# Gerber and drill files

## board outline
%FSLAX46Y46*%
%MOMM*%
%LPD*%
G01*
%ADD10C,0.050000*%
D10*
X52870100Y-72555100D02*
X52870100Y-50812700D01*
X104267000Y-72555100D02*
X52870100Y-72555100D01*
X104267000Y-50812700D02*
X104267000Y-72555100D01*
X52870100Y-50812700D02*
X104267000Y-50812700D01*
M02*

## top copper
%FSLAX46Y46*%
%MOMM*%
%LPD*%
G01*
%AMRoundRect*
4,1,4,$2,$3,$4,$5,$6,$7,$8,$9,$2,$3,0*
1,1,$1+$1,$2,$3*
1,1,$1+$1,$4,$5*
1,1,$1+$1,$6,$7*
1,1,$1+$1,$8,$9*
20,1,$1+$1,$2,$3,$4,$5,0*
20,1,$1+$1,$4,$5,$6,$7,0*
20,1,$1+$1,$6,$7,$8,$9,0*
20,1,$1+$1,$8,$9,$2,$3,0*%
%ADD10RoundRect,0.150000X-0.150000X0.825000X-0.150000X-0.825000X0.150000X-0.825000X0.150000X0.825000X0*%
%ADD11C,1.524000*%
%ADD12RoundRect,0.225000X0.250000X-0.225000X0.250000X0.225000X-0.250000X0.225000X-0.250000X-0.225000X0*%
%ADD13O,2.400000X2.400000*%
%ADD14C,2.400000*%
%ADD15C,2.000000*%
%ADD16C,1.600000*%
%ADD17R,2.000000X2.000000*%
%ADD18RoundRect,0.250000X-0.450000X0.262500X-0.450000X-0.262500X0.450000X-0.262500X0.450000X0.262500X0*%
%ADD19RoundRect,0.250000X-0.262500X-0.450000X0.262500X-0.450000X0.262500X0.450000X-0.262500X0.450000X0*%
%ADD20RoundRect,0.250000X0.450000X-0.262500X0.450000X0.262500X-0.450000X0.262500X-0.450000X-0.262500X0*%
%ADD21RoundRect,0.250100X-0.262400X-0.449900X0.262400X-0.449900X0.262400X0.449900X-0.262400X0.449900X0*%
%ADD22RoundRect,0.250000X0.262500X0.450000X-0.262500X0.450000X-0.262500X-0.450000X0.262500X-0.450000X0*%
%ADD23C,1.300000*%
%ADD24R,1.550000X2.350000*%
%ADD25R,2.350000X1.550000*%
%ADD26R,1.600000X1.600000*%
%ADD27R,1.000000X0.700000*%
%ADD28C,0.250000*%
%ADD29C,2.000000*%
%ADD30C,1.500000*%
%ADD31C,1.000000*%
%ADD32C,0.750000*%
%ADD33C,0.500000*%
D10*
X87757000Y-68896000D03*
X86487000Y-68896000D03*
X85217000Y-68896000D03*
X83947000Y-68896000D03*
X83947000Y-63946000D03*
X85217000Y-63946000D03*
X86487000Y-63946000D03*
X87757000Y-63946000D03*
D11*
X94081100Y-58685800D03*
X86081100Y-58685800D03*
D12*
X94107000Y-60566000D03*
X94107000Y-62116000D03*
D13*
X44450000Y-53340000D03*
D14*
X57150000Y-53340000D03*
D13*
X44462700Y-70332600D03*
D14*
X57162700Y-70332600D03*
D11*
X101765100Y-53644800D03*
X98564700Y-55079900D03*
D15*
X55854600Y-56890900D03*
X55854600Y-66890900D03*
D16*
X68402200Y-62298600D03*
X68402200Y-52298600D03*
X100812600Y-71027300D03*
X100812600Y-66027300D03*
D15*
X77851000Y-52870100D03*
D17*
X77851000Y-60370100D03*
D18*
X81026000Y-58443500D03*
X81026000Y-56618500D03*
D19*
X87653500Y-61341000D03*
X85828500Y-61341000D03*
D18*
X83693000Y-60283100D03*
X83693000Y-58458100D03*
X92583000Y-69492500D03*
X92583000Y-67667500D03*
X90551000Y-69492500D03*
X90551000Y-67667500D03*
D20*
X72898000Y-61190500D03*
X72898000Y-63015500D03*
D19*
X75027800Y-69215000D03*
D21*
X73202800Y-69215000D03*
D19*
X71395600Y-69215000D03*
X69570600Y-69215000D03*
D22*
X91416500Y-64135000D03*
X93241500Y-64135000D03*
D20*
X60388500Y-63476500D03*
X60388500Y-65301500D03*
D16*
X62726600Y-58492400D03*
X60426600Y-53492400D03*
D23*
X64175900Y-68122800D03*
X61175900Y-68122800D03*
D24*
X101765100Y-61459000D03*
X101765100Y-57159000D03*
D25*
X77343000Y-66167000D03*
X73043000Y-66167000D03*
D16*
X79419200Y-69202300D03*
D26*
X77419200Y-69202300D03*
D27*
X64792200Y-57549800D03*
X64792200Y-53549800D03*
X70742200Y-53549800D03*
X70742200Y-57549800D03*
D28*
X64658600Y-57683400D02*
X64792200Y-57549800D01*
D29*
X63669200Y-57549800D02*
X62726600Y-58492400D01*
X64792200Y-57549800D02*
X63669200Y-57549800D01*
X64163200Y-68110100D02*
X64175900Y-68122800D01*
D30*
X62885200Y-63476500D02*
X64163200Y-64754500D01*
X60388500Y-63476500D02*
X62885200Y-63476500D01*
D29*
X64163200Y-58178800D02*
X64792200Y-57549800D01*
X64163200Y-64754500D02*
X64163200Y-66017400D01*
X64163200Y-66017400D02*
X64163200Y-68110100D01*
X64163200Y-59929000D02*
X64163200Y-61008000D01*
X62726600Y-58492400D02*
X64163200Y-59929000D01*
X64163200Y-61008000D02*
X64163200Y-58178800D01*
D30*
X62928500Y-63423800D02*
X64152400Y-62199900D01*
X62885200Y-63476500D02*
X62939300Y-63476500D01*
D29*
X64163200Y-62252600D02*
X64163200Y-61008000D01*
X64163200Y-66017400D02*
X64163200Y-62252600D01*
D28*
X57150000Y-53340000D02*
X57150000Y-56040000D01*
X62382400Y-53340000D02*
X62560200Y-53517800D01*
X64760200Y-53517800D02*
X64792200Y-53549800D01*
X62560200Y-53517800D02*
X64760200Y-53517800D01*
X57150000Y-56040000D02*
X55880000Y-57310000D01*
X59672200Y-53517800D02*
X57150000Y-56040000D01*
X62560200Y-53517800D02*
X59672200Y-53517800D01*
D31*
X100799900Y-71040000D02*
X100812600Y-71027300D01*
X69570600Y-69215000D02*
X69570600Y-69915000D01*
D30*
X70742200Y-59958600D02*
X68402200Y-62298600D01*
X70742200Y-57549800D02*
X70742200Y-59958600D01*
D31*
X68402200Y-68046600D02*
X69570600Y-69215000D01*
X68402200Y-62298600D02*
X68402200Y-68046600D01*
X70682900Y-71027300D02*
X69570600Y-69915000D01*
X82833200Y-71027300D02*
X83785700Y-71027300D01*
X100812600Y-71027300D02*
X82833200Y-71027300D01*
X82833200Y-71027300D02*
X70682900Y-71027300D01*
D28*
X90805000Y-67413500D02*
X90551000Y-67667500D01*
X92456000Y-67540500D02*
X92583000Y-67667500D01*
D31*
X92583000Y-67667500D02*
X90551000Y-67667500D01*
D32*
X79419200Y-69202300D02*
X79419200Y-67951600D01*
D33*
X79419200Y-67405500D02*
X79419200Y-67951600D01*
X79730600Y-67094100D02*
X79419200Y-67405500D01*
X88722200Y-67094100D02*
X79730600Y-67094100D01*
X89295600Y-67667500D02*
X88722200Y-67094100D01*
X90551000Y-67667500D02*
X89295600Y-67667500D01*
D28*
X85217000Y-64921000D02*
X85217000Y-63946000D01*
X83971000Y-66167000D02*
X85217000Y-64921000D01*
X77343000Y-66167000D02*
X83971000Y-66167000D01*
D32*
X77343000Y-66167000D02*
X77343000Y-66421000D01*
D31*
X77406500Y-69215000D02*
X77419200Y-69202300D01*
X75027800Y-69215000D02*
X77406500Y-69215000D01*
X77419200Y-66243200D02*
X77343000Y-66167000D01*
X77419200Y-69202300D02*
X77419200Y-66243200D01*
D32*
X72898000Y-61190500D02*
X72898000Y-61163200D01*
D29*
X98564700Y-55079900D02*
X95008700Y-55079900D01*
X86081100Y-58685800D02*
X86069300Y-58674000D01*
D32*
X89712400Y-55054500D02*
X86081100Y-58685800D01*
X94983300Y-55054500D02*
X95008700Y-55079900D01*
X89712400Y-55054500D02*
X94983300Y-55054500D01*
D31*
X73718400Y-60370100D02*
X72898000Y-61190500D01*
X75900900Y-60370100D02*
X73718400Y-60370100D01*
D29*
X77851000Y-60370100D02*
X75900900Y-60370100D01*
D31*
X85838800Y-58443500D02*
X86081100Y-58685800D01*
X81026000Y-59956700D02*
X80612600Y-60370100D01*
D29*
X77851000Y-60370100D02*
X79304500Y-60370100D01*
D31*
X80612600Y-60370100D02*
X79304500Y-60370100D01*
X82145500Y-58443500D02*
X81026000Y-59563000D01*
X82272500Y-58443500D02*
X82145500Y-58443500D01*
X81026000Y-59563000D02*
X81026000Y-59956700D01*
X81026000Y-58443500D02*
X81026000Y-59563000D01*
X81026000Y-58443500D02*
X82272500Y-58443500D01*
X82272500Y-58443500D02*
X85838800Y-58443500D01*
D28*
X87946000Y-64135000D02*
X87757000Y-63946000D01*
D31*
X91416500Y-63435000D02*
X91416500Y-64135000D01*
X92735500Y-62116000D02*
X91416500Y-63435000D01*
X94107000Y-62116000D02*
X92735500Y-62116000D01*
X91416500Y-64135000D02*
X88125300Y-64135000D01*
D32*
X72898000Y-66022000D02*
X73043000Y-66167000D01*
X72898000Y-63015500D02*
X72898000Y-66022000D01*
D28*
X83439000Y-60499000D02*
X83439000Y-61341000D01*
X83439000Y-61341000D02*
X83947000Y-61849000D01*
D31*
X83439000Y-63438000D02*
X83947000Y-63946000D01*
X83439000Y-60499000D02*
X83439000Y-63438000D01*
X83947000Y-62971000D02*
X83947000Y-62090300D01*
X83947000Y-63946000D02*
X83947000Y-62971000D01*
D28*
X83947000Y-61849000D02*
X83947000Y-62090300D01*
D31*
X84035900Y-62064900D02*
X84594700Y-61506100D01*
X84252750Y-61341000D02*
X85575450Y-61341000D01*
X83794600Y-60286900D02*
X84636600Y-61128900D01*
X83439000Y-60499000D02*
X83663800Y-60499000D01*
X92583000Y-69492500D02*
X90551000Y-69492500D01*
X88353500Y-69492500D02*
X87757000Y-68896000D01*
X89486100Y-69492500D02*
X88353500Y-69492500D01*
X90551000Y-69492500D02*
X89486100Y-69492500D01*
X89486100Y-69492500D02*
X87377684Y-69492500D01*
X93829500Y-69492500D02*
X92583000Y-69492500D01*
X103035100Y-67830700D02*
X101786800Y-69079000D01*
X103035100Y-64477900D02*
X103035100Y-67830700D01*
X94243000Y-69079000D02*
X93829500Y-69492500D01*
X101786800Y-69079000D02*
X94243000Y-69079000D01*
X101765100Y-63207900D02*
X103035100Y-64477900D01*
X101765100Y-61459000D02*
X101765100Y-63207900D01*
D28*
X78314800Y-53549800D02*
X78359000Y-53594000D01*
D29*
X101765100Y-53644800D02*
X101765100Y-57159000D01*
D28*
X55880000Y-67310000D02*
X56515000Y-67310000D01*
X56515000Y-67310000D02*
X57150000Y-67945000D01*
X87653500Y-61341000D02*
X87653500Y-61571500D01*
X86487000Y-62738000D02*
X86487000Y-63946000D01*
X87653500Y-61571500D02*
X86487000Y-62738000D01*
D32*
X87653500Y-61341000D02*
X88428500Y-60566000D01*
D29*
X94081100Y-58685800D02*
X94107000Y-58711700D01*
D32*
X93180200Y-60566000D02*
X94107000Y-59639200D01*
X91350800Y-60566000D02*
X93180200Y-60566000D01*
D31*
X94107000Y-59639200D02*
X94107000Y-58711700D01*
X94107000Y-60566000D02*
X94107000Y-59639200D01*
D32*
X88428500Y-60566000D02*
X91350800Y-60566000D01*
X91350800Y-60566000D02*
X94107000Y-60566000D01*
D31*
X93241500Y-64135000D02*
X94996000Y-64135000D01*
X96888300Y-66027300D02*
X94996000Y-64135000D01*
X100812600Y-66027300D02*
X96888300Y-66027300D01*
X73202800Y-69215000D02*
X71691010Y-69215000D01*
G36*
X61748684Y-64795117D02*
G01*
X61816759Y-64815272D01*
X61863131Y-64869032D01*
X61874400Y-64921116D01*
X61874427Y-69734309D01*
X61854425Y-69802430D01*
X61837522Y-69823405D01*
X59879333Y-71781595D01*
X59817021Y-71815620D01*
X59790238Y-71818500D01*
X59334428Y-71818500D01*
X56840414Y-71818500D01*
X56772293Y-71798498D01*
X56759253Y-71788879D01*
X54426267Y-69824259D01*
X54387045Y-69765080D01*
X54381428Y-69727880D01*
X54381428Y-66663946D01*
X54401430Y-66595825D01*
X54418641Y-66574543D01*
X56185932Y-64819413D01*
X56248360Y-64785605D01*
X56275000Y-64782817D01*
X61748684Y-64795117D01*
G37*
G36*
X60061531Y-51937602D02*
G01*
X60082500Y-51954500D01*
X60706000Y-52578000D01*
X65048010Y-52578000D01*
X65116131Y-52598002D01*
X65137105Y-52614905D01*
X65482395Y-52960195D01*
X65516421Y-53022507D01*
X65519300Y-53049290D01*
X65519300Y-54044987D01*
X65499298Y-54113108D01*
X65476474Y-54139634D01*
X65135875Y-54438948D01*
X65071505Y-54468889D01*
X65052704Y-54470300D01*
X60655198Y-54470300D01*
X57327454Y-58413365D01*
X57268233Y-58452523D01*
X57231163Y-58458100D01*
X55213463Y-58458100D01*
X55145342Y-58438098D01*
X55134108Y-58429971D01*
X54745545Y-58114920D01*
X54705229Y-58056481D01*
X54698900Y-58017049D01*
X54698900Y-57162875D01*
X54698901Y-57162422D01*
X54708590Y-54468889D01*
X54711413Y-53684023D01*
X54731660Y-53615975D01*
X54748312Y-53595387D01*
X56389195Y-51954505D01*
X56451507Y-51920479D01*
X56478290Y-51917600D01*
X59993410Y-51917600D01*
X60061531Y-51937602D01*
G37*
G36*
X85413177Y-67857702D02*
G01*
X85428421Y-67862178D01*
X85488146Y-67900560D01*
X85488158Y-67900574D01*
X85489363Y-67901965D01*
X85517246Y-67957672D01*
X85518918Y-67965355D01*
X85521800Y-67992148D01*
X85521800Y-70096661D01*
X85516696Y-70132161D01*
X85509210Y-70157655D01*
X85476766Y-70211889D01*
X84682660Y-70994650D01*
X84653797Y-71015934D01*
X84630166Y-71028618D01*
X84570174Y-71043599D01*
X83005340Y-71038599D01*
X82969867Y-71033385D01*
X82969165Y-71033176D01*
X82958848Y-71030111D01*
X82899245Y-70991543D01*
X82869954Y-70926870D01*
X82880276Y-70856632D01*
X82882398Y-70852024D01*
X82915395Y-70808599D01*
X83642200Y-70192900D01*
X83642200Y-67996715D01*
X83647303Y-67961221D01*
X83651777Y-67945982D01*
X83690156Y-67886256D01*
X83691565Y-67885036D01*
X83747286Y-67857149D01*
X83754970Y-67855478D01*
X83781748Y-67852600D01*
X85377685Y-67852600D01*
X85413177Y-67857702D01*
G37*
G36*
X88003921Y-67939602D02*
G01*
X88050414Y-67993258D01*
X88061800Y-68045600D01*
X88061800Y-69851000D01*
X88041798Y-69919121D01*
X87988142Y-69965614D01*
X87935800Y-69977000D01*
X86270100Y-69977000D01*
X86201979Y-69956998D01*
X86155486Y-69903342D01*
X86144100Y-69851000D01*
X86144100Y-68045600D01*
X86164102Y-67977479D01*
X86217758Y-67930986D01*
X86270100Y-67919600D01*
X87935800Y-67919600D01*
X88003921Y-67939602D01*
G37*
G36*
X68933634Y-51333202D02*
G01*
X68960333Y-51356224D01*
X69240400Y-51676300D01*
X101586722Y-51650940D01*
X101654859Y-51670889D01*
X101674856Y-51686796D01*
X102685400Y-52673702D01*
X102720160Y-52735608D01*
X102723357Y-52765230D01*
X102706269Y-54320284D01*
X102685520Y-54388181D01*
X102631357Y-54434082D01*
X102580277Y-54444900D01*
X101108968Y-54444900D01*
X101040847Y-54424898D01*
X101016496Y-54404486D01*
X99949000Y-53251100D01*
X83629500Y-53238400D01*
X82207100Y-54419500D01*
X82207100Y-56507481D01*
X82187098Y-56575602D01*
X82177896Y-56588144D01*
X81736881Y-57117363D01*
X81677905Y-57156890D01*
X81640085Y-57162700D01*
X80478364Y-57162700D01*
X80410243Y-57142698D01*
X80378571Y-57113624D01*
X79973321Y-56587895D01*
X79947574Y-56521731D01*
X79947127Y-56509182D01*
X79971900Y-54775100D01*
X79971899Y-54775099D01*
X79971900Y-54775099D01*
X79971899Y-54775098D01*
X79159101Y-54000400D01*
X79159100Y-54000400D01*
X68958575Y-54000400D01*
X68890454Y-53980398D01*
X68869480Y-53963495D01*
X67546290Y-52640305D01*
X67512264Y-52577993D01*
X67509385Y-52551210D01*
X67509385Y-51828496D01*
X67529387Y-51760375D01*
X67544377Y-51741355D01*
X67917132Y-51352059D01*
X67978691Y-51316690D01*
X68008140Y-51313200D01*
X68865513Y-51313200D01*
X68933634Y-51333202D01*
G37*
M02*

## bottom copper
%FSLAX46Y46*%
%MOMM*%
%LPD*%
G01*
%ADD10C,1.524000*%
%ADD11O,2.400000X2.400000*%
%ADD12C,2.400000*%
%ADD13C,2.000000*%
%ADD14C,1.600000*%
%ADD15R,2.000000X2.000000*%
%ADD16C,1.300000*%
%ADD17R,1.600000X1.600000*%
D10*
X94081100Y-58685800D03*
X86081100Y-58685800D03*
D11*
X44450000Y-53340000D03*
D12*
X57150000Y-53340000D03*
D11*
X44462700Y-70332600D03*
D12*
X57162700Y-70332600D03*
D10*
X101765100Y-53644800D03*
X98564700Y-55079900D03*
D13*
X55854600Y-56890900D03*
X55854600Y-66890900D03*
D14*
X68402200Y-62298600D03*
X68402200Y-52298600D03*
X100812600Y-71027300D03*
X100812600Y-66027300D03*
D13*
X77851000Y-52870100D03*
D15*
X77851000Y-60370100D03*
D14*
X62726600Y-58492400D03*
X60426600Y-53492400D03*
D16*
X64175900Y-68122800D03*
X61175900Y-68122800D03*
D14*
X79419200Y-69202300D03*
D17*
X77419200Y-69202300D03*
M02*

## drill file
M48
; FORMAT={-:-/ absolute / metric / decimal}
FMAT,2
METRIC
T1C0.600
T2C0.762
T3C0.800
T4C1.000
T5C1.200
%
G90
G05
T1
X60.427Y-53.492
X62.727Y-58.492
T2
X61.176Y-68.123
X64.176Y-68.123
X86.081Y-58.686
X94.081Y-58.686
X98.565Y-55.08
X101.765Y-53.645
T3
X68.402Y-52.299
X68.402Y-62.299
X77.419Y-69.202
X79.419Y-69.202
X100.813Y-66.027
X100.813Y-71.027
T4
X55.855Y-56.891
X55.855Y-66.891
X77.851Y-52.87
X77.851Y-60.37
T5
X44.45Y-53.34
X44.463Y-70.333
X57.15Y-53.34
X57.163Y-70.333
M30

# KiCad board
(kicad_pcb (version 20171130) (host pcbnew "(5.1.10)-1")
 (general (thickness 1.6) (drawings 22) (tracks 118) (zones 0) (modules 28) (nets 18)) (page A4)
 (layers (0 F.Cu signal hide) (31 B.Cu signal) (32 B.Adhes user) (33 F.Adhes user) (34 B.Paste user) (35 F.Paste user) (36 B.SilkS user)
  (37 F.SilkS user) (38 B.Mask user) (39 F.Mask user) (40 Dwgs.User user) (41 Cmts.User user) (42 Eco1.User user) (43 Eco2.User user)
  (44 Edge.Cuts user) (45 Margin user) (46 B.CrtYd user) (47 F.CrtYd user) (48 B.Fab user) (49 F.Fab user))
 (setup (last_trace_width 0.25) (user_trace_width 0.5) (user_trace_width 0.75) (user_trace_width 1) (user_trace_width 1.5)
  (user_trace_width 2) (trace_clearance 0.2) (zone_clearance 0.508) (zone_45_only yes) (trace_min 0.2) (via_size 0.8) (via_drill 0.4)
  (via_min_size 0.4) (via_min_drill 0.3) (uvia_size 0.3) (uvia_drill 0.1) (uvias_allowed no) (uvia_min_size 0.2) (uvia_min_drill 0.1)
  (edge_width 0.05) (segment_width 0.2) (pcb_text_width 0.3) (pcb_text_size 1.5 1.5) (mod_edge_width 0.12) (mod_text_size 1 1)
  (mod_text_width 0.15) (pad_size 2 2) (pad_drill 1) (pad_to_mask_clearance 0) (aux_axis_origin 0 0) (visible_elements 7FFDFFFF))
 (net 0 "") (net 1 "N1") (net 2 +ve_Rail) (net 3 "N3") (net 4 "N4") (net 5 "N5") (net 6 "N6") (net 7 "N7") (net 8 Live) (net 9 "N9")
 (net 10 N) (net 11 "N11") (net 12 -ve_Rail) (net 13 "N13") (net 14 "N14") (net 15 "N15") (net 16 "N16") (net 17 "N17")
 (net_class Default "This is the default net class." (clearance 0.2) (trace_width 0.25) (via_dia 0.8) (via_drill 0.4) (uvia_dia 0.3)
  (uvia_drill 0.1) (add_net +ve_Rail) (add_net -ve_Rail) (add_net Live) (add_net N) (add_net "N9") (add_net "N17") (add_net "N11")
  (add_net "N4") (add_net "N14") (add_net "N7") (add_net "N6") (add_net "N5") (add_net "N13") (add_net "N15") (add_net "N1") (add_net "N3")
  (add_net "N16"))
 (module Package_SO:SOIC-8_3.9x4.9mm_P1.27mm (layer F.Cu) (at 85.852 66.421 270)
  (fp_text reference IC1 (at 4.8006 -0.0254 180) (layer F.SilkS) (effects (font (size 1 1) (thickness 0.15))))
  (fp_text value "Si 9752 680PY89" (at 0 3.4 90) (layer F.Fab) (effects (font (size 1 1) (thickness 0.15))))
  (pad 8 smd roundrect (at 2.475 -1.905 270) (size 1.95 0.6) (layers F.Cu F.Paste F.Mask) (roundrect_rratio 0.25) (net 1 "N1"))
  (pad 7 smd roundrect (at 2.475 -0.635 270) (size 1.95 0.6) (layers F.Cu F.Paste F.Mask) (roundrect_rratio 0.25) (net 1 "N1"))
  (pad 6 smd roundrect (at 2.475 0.635 270) (size 1.95 0.6) (layers F.Cu F.Paste F.Mask) (roundrect_rratio 0.25) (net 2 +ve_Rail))
  (pad 5 smd roundrect (at 2.475 1.905 270) (size 1.95 0.6) (layers F.Cu F.Paste F.Mask) (roundrect_rratio 0.25) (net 2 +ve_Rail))
  (pad 4 smd roundrect (at -2.475 1.905 270) (size 1.95 0.6) (layers F.Cu F.Paste F.Mask) (roundrect_rratio 0.25) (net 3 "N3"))
  (pad 3 smd roundrect (at -2.475 0.635 270) (size 1.95 0.6) (layers F.Cu F.Paste F.Mask) (roundrect_rratio 0.25) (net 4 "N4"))
  (pad 2 smd roundrect (at -2.475 -0.635 270) (size 1.95 0.6) (layers F.Cu F.Paste F.Mask) (roundrect_rratio 0.25) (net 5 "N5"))
  (pad 1 smd roundrect (at -2.475 -1.905 270) (size 1.95 0.6) (layers F.Cu F.Paste F.Mask) (roundrect_rratio 0.25) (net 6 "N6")))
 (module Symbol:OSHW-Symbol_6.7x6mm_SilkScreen (layer B.Cu) (at 71.2851 68.5673 180)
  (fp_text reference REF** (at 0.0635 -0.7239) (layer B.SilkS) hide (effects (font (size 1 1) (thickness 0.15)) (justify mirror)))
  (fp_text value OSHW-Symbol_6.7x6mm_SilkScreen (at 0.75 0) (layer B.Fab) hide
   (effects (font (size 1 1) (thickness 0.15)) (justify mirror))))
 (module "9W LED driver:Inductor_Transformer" (layer B.Cu) (at 90.0811 64.1858)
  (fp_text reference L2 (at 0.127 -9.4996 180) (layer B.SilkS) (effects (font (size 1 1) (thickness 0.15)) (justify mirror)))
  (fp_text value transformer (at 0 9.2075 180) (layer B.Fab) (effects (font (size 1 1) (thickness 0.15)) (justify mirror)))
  (pad 2 thru_hole circle (at 4 -5.5) (size 1.524 1.524) (drill 0.762) (layers *.Cu *.Mask) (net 5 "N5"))
  (pad 1 thru_hole circle (at -4 -5.5) (size 1.524 1.524) (drill 0.762) (layers *.Cu *.Mask) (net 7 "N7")))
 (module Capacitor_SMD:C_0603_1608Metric (layer F.Cu) (at 94.107 61.341 90)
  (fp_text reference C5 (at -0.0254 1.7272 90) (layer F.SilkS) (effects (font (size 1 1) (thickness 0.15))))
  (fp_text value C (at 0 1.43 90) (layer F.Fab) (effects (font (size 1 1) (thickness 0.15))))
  (pad 2 smd roundrect (at 0.775 0 90) (size 0.9 0.95) (layers F.Cu F.Paste F.Mask) (roundrect_rratio 0.25) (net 5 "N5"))
  (pad 1 smd roundrect (at -0.775 0 90) (size 0.9 0.95) (layers F.Cu F.Paste F.Mask) (roundrect_rratio 0.25) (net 6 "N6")))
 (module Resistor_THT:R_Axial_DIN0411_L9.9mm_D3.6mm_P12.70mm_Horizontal (layer B.Cu) (at 57.15 53.34 180)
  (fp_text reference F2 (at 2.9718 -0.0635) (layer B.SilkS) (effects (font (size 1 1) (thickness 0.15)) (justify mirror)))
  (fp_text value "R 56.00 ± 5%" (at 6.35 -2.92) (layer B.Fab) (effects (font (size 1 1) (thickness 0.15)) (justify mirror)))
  (pad 2 thru_hole oval (at 12.7 0 180) (size 2.4 2.4) (drill 1.2) (layers *.Cu *.Mask) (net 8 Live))
  (pad 1 thru_hole circle (at 0 0 180) (size 2.4 2.4) (drill 1.2) (layers *.Cu *.Mask) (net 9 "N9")))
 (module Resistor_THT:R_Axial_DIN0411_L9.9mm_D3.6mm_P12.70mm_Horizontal (layer B.Cu) (at 57.1627 70.3326 180)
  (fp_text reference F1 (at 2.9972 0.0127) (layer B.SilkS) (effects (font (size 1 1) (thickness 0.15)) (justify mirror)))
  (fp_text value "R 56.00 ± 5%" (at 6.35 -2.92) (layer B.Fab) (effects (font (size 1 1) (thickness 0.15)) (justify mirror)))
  (pad 2 thru_hole oval (at 12.7 0 180) (size 2.4 2.4) (drill 1.2) (layers *.Cu *.Mask) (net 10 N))
  (pad 1 thru_hole circle (at 0 0 180) (size 2.4 2.4) (drill 1.2) (layers *.Cu *.Mask) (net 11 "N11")))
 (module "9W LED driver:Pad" (layer F.Cu) (at 101.7651 53.6448)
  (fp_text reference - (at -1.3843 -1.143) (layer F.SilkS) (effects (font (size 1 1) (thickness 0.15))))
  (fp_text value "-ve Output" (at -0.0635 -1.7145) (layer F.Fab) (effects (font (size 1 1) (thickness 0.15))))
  (pad 1 thru_hole circle (at 0 0) (size 1.524 1.524) (drill 0.762) (layers *.Cu *.Mask) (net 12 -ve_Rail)))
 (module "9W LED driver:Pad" (layer F.Cu) (at 98.5647 55.0799)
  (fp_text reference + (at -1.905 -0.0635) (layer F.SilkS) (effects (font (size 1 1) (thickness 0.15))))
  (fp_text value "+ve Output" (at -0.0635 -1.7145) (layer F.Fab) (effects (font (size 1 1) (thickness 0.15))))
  (pad 1 thru_hole circle (at 0 0) (size 1.524 1.524) (drill 0.762) (layers *.Cu *.Mask) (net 7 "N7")))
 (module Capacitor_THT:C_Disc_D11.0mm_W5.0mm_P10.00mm (layer B.Cu) (at 55.8546 66.8909 90)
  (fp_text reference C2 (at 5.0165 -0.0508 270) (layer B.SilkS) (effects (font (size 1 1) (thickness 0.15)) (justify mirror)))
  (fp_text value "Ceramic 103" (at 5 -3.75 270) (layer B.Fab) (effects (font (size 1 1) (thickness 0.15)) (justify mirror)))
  (pad 2 thru_hole circle (at 10 0 90) (size 2 2) (drill 1) (layers *.Cu *.Mask) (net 9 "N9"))
  (pad 1 thru_hole circle (at 0 0 90) (size 2 2) (drill 1) (layers *.Cu *.Mask) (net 11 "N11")))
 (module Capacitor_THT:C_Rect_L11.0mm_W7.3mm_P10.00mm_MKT (layer B.Cu) (at 68.4022 52.2986 270)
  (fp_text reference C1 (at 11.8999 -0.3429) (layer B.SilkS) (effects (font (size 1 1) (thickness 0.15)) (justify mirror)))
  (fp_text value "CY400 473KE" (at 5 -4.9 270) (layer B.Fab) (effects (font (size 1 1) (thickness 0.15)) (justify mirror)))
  (pad 2 thru_hole circle (at 10 0 270) (size 1.6 1.6) (drill 0.8) (layers *.Cu *.Mask) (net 2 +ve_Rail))
  (pad 1 thru_hole circle (at 0 0 270) (size 1.6 1.6) (drill 0.8) (layers *.Cu *.Mask) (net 12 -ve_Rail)))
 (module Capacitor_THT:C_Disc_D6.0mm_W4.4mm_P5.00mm (layer B.Cu) (at 100.8126 66.0273 270)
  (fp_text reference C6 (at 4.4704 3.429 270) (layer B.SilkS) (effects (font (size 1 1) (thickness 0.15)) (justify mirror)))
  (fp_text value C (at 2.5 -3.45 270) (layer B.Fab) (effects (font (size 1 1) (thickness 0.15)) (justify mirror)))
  (pad 2 thru_hole circle (at 5 0 270) (size 1.6 1.6) (drill 0.8) (layers *.Cu *.Mask) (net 2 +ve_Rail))
  (pad 1 thru_hole circle (at 0 0 270) (size 1.6 1.6) (drill 0.8) (layers *.Cu *.Mask) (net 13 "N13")))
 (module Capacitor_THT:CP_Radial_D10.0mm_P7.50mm (layer B.Cu) (at 77.851 60.3701 90)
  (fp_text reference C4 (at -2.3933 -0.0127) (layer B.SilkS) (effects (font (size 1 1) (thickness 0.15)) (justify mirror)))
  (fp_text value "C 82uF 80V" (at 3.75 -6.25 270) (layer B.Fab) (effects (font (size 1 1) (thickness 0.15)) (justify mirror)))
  (pad 2 thru_hole circle (at 7.5 0 90) (size 2 2) (drill 1) (layers *.Cu *.Mask) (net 12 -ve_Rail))
  (pad 1 thru_hole rect (at 0 0 90) (size 2 2) (drill 1) (layers *.Cu *.Mask F.Paste) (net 7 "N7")))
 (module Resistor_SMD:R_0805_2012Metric (layer F.Cu) (at 81.026 57.531 270)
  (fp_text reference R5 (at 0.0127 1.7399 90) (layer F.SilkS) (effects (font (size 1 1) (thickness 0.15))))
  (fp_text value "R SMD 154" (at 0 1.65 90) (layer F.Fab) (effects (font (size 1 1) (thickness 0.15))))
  (pad 2 smd roundrect (at 0.9125 0 270) (size 1.025 1.4) (layers F.Cu F.Paste F.Mask) (roundrect_rratio 0.243902) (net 7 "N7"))
  (pad 1 smd roundrect (at -0.9125 0 270) (size 1.025 1.4) (layers F.Cu F.Paste F.Mask) (roundrect_rratio 0.243902) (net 12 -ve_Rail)))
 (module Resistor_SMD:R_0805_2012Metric (layer F.Cu) (at 86.741 61.341)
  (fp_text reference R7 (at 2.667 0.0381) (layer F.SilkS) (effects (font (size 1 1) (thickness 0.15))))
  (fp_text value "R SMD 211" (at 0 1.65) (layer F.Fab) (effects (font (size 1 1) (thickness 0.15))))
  (pad 2 smd roundrect (at 0.9125 0) (size 1.025 1.4) (layers F.Cu F.Paste F.Mask) (roundrect_rratio 0.243902) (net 5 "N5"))
  (pad 1 smd roundrect (at -0.9125 0) (size 1.025 1.4) (layers F.Cu F.Paste F.Mask) (roundrect_rratio 0.243902) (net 3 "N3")))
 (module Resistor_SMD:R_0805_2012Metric (layer F.Cu) (at 83.693 59.3706 270)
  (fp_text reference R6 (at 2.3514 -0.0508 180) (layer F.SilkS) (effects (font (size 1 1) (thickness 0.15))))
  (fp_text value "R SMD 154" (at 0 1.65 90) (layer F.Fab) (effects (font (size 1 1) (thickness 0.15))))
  (pad 2 smd roundrect (at 0.9125 0 270) (size 1.025 1.4) (layers F.Cu F.Paste F.Mask) (roundrect_rratio 0.243902) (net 3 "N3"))
  (pad 1 smd roundrect (at -0.9125 0 270) (size 1.025 1.4) (layers F.Cu F.Paste F.Mask) (roundrect_rratio 0.243902) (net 7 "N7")))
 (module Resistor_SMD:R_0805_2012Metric (layer F.Cu) (at 92.583 68.58 270)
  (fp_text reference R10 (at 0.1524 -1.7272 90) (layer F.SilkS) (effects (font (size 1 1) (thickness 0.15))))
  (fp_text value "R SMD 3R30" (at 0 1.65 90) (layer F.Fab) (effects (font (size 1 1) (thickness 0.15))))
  (pad 2 smd roundrect (at 0.9125 0 270) (size 1.025 1.4) (layers F.Cu F.Paste F.Mask) (roundrect_rratio 0.243902) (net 1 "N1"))
  (pad 1 smd roundrect (at -0.9125 0 270) (size 1.025 1.4) (layers F.Cu F.Paste F.Mask) (roundrect_rratio 0.243902) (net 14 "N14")))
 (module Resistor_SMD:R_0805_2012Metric (layer F.Cu) (at 90.551 68.58 270)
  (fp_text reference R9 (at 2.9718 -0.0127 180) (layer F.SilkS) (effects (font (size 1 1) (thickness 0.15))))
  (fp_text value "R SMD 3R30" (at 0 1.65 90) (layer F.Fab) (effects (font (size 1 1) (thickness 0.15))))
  (pad 2 smd roundrect (at 0.9125 0 270) (size 1.025 1.4) (layers F.Cu F.Paste F.Mask) (roundrect_rratio 0.243902) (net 1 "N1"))
  (pad 1 smd roundrect (at -0.9125 0 270) (size 1.025 1.4) (layers F.Cu F.Paste F.Mask) (roundrect_rratio 0.243902) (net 14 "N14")))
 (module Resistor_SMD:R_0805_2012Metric (layer F.Cu) (at 72.898 62.103 90)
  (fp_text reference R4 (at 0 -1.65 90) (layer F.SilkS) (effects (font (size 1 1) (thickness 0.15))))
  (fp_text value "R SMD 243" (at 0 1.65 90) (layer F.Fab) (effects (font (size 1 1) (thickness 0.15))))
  (pad 2 smd roundrect (at 0.9125 0 90) (size 1.025 1.4) (layers F.Cu F.Paste F.Mask) (roundrect_rratio 0.243902) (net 7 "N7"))
  (pad 1 smd roundrect (at -0.9125 0 90) (size 1.025 1.4) (layers F.Cu F.Paste F.Mask) (roundrect_rratio 0.243902) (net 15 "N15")))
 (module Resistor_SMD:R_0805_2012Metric (layer F.Cu) (at 74.1153 69.215)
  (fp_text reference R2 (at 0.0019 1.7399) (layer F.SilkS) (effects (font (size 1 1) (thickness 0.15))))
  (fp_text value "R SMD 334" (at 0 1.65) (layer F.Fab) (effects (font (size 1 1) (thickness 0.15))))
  (pad 2 smd roundrect (at 0.9125 0) (size 1.025 1.4) (layers F.Cu F.Paste F.Mask) (roundrect_rratio 0.243902) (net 4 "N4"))
  (pad 1 smd roundrect (at -0.9125 0) (size 1.025 1.4) (layers F.Cu F.Paste F.Mask) (roundrect_rratio 0.244) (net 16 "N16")))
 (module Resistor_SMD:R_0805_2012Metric (layer F.Cu) (at 70.4831 69.215)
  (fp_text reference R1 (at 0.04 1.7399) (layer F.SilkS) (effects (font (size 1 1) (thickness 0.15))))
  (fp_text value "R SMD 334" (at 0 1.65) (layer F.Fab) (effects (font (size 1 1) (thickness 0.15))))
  (pad 2 smd roundrect (at 0.9125 0) (size 1.025 1.4) (layers F.Cu F.Paste F.Mask) (roundrect_rratio 0.243902) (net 16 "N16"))
  (pad 1 smd roundrect (at -0.9125 0) (size 1.025 1.4) (layers F.Cu F.Paste F.Mask) (roundrect_rratio 0.243902) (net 2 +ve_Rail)))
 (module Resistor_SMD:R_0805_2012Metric (layer F.Cu) (at 92.329 64.135 180)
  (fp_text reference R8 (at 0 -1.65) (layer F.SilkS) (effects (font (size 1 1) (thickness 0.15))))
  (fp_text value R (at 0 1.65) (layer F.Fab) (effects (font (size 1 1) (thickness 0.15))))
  (pad 2 smd roundrect (at 0.9125 0 180) (size 1.025 1.4) (layers F.Cu F.Paste F.Mask) (roundrect_rratio 0.243902) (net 6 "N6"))
  (pad 1 smd roundrect (at -0.9125 0 180) (size 1.025 1.4) (layers F.Cu F.Paste F.Mask) (roundrect_rratio 0.243902) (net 13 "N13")))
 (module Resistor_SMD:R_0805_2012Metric (layer F.Cu) (at 60.3885 64.389 90)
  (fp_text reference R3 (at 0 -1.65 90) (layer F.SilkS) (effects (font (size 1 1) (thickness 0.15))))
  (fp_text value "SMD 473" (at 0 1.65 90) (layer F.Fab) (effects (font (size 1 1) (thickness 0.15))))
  (pad 2 smd roundrect (at 0.9125 0 90) (size 1.025 1.4) (layers F.Cu F.Paste F.Mask) (roundrect_rratio 0.243902) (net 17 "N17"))
  (pad 1 smd roundrect (at -0.9125 0 90) (size 1.025 1.4) (layers F.Cu F.Paste F.Mask) (roundrect_rratio 0.243902) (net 11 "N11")))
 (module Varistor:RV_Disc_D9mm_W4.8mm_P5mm (layer B.Cu) (at 60.4266 53.4924 270)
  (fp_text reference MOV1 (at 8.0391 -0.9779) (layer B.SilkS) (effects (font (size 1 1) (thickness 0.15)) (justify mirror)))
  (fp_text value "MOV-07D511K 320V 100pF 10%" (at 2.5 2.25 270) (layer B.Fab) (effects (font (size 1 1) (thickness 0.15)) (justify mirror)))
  (pad 2 thru_hole circle (at 5 -2.3 270) (size 1.6 1.6) (drill 0.6) (layers *.Cu *.Mask) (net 17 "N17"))
  (pad 1 thru_hole circle (at 0 0 270) (size 1.6 1.6) (drill 0.6) (layers *.Cu *.Mask) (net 9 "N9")))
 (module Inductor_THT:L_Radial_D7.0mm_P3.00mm (layer B.Cu) (at 61.1759 68.1228)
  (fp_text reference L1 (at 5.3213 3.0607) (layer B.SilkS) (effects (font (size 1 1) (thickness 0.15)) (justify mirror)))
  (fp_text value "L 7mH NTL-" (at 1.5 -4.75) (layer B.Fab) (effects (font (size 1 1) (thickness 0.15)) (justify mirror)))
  (pad 2 thru_hole circle (at 3 0) (size 1.3 1.3) (drill 0.762) (layers *.Cu *.Mask) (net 17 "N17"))
  (pad 1 thru_hole circle (at 0 0) (size 1.3 1.3) (drill 0.762) (layers *.Cu *.Mask B.Adhes) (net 11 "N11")))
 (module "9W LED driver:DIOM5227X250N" (layer F.Cu) (at 101.7651 59.309 90)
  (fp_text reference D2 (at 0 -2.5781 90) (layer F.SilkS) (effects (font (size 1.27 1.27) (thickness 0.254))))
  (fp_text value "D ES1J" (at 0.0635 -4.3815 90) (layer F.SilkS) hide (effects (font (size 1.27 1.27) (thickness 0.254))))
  (pad 1 smd rect (at -2.15 0 180) (size 1.55 2.35) (layers F.Cu F.Paste F.Mask) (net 1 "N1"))
  (pad 2 smd rect (at 2.15 0 180) (size 1.55 2.35) (layers F.Cu F.Paste F.Mask) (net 12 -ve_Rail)))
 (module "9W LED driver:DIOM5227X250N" (layer F.Cu) (at 75.193 66.167 180)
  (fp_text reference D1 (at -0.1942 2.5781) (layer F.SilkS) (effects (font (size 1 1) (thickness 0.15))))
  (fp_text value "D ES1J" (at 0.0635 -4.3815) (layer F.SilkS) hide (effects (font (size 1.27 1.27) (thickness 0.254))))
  (pad 1 smd rect (at -2.15 0 270) (size 1.55 2.35) (layers F.Cu F.Paste F.Mask) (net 4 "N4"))
  (pad 2 smd rect (at 2.15 0 270) (size 1.55 2.35) (layers F.Cu F.Paste F.Mask) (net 15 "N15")))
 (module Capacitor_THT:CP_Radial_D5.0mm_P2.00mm (layer B.Cu) (at 77.4192 69.2023)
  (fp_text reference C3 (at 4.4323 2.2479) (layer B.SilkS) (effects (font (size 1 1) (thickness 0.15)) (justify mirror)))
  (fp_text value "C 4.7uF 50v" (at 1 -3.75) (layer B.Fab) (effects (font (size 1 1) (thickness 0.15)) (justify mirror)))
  (pad 2 thru_hole circle (at 2 0) (size 1.6 1.6) (drill 0.8) (layers *.Cu *.Mask) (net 14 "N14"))
  (pad 1 thru_hole rect (at 0 0) (size 1.6 1.6) (drill 0.8) (layers *.Cu *.Mask) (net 4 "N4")))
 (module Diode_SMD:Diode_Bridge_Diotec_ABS (layer F.Cu) (at 67.7672 55.5498 180)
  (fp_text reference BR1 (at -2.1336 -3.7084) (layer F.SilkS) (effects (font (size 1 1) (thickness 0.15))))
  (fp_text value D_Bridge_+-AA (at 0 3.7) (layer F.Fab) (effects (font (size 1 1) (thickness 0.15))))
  (pad 4 smd rect (at 2.975 -2 180) (size 1 0.7) (layers F.Cu F.Paste F.Mask) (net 17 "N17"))
  (pad 3 smd rect (at 2.975 2 180) (size 1 0.7) (layers F.Cu F.Paste F.Mask) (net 9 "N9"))
  (pad 2 smd rect (at -2.975 2 180) (size 1 0.7) (layers F.Cu F.Paste F.Mask) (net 12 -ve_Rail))
  (pad 1 smd rect (at -2.975 -2 180) (size 1 0.7) (layers F.Cu F.Paste F.Mask) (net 2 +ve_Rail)))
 (gr_line (start 52.8701 72.5551) (end 52.8701 50.8127) (layer Edge.Cuts) (width 0.05))
 (gr_line (start 104.267 72.5551) (end 52.8701 72.5551) (layer Edge.Cuts) (width 0.05))
 (gr_line (start 104.267 50.8127) (end 104.267 72.5551) (layer Edge.Cuts) (width 0.05))
 (gr_line (start 52.8701 50.8127) (end 104.267 50.8127) (layer Edge.Cuts) (width 0.05))
 (segment (start 64.6586 57.6834) (end 64.7922 57.5498) (width 0.25) (layer F.Cu) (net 17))
 (segment (start 63.6692 57.5498) (end 62.7266 58.4924) (width 2) (layer F.Cu) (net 17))
 (segment (start 64.7922 57.5498) (end 63.6692 57.5498) (width 2) (layer F.Cu) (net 17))
 (segment (start 64.1632 68.1101) (end 64.1759 68.1228) (width 2) (layer F.Cu) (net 17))
 (segment (start 62.8852 63.4765) (end 64.1632 64.7545) (width 1.5) (layer F.Cu) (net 17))
 (segment (start 60.3885 63.4765) (end 62.8852 63.4765) (width 1.5) (layer F.Cu) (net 17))
 (segment (start 64.1632 58.1788) (end 64.7922 57.5498) (width 2) (layer F.Cu) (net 17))
 (segment (start 64.1632 64.7545) (end 64.1632 66.0174) (width 2) (layer F.Cu) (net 17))
 (segment (start 64.1632 66.0174) (end 64.1632 68.1101) (width 2) (layer F.Cu) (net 17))
 (segment (start 64.1632 59.929) (end 64.1632 61.008) (width 2) (layer F.Cu) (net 17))
 (segment (start 62.7266 58.4924) (end 64.1632 59.929) (width 2) (layer F.Cu) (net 17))
 (segment (start 64.1632 61.008) (end 64.1632 58.1788) (width 2) (layer F.Cu) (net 17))
 (segment (start 62.9285 63.4238) (end 64.1524 62.1999) (width 1.5) (layer F.Cu) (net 17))
 (segment (start 62.8852 63.4765) (end 62.9393 63.4765) (width 1.5) (layer F.Cu) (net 17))
 (segment (start 64.1632 62.2526) (end 64.1632 61.008) (width 2) (layer F.Cu) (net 17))
 (segment (start 64.1632 66.0174) (end 64.1632 62.2526) (width 2) (layer F.Cu) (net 17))
 (segment (start 57.15 53.34) (end 57.15 56.04) (width 0.25) (layer F.Cu) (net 9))
 (segment (start 62.3824 53.34) (end 62.5602 53.5178) (width 0.25) (layer F.Cu) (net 9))
 (segment (start 64.7602 53.5178) (end 64.7922 53.5498) (width 0.25) (layer F.Cu) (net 9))
 (segment (start 62.5602 53.5178) (end 64.7602 53.5178) (width 0.25) (layer F.Cu) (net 9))
 (segment (start 57.15 56.04) (end 55.88 57.31) (width 0.25) (layer F.Cu) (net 9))
 (segment (start 59.6722 53.5178) (end 57.15 56.04) (width 0.25) (layer F.Cu) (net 9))
 (segment (start 62.5602 53.5178) (end 59.6722 53.5178) (width 0.25) (layer F.Cu) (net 9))
 (segment (start 100.7999 71.04) (end 100.8126 71.0273) (width 1) (layer F.Cu) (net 2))
 (segment (start 69.5706 69.215) (end 69.5706 69.915) (width 1) (layer F.Cu) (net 2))
 (segment (start 70.7422 59.9586) (end 68.4022 62.2986) (width 1.5) (layer F.Cu) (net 2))
 (segment (start 70.7422 57.5498) (end 70.7422 59.9586) (width 1.5) (layer F.Cu) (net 2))
 (segment (start 68.4022 68.0466) (end 69.5706 69.215) (width 1) (layer F.Cu) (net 2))
 (segment (start 68.4022 62.2986) (end 68.4022 68.0466) (width 1) (layer F.Cu) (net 2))
 (segment (start 70.6829 71.0273) (end 69.5706 69.915) (width 1) (layer F.Cu) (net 2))
 (segment (start 82.8332 71.0273) (end 83.7857 71.0273) (width 1) (layer F.Cu) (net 2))
 (segment (start 100.8126 71.0273) (end 82.8332 71.0273) (width 1) (layer F.Cu) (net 2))
 (segment (start 82.8332 71.0273) (end 70.6829 71.0273) (width 1) (layer F.Cu) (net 2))
 (segment (start 90.805 67.4135) (end 90.551 67.6675) (width 0.25) (layer F.Cu) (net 14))
 (segment (start 92.456 67.5405) (end 92.583 67.6675) (width 0.25) (layer F.Cu) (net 14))
 (segment (start 92.583 67.6675) (end 90.551 67.6675) (width 1) (layer F.Cu) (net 14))
 (segment (start 79.4192 69.2023) (end 79.4192 67.9516) (width 0.75) (layer F.Cu) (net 14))
 (segment (start 79.4192 67.4055) (end 79.4192 67.9516) (width 0.5) (layer F.Cu) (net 14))
 (segment (start 79.7306 67.0941) (end 79.4192 67.4055) (width 0.5) (layer F.Cu) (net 14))
 (segment (start 88.7222 67.0941) (end 79.7306 67.0941) (width 0.5) (layer F.Cu) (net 14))
 (segment (start 89.2956 67.6675) (end 88.7222 67.0941) (width 0.5) (layer F.Cu) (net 14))
 (segment (start 90.551 67.6675) (end 89.2956 67.6675) (width 0.5) (layer F.Cu) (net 14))
 (segment (start 85.217 64.921) (end 85.217 63.946) (width 0.25) (layer F.Cu) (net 4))
 (segment (start 83.971 66.167) (end 85.217 64.921) (width 0.25) (layer F.Cu) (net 4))
 (segment (start 77.343 66.167) (end 83.971 66.167) (width 0.25) (layer F.Cu) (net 4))
 (segment (start 77.343 66.167) (end 77.343 66.421) (width 0.75) (layer F.Cu) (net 4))
 (segment (start 77.4065 69.215) (end 77.4192 69.2023) (width 1) (layer F.Cu) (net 4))
 (segment (start 75.0278 69.215) (end 77.4065 69.215) (width 1) (layer F.Cu) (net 4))
 (segment (start 77.4192 66.2432) (end 77.343 66.167) (width 1) (layer F.Cu) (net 4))
 (segment (start 77.4192 69.2023) (end 77.4192 66.2432) (width 1) (layer F.Cu) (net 4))
 (segment (start 72.898 61.1905) (end 72.898 61.1632) (width 0.75) (layer F.Cu) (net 7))
 (segment (start 98.5647 55.0799) (end 95.0087 55.0799) (width 2) (layer F.Cu) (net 7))
 (segment (start 86.0811 58.6858) (end 86.0693 58.674) (width 2) (layer F.Cu) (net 7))
 (segment (start 89.7124 55.0545) (end 86.0811 58.6858) (width 0.75) (layer F.Cu) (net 7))
 (segment (start 94.9833 55.0545) (end 95.0087 55.0799) (width 0.75) (layer F.Cu) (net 7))
 (segment (start 89.7124 55.0545) (end 94.9833 55.0545) (width 0.75) (layer F.Cu) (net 7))
 (segment (start 73.7184 60.3701) (end 72.898 61.1905) (width 1) (layer F.Cu) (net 7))
 (segment (start 75.9009 60.3701) (end 73.7184 60.3701) (width 1) (layer F.Cu) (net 7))
 (segment (start 77.851 60.3701) (end 75.9009 60.3701) (width 2) (layer F.Cu) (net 7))
 (segment (start 85.8388 58.4435) (end 86.0811 58.6858) (width 1) (layer F.Cu) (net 7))
 (segment (start 81.026 59.9567) (end 80.6126 60.3701) (width 1) (layer F.Cu) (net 7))
 (segment (start 77.851 60.3701) (end 79.3045 60.3701) (width 2) (layer F.Cu) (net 7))
 (segment (start 80.6126 60.3701) (end 79.3045 60.3701) (width 1) (layer F.Cu) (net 7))
 (segment (start 82.1455 58.4435) (end 81.026 59.563) (width 1) (layer F.Cu) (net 7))
 (segment (start 82.2725 58.4435) (end 82.1455 58.4435) (width 1) (layer F.Cu) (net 7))
 (segment (start 81.026 59.563) (end 81.026 59.9567) (width 1) (layer F.Cu) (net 7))
 (segment (start 81.026 58.4435) (end 81.026 59.563) (width 1) (layer F.Cu) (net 7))
 (segment (start 81.026 58.4435) (end 82.2725 58.4435) (width 1) (layer F.Cu) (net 7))
 (segment (start 82.2725 58.4435) (end 85.8388 58.4435) (width 1) (layer F.Cu) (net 7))
 (segment (start 87.946 64.135) (end 87.757 63.946) (width 0.25) (layer F.Cu) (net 6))
 (segment (start 91.4165 63.435) (end 91.4165 64.135) (width 1) (layer F.Cu) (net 6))
 (segment (start 92.7355 62.116) (end 91.4165 63.435) (width 1) (layer F.Cu) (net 6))
 (segment (start 94.107 62.116) (end 92.7355 62.116) (width 1) (layer F.Cu) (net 6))
 (segment (start 91.4165 64.135) (end 88.1253 64.135) (width 1) (layer F.Cu) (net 6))
 (segment (start 72.898 66.022) (end 73.043 66.167) (width 0.75) (layer F.Cu) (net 15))
 (segment (start 72.898 63.0155) (end 72.898 66.022) (width 0.75) (layer F.Cu) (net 15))
 (segment (start 83.439 60.499) (end 83.439 61.341) (width 0.25) (layer F.Cu) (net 3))
 (segment (start 83.439 61.341) (end 83.947 61.849) (width 0.25) (layer F.Cu) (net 3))
 (segment (start 83.439 63.438) (end 83.947 63.946) (width 1) (layer F.Cu) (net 3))
 (segment (start 83.439 60.499) (end 83.439 63.438) (width 1) (layer F.Cu) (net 3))
 (segment (start 83.947 62.971) (end 83.947 62.0903) (width 1) (layer F.Cu) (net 3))
 (segment (start 83.947 63.946) (end 83.947 62.971) (width 1) (layer F.Cu) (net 3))
 (segment (start 83.947 61.849) (end 83.947 62.0903) (width 0.25) (layer F.Cu) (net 3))
 (segment (start 84.0359 62.0649) (end 84.5947 61.5061) (width 1) (layer F.Cu) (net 3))
 (segment (start 84.25275 61.341) (end 85.57545 61.341) (width 1) (layer F.Cu) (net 3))
 (segment (start 83.7946 60.2869) (end 84.6366 61.1289) (width 1) (layer F.Cu) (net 3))
 (segment (start 83.439 60.499) (end 83.6638 60.499) (width 1) (layer F.Cu) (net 3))
 (segment (start 92.583 69.4925) (end 90.551 69.4925) (width 1) (layer F.Cu) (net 1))
 (segment (start 88.3535 69.4925) (end 87.757 68.896) (width 1) (layer F.Cu) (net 1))
 (segment (start 89.4861 69.4925) (end 88.3535 69.4925) (width 1) (layer F.Cu) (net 1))
 (segment (start 90.551 69.4925) (end 89.4861 69.4925) (width 1) (layer F.Cu) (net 1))
 (segment (start 89.4861 69.4925) (end 87.377684 69.4925) (width 1) (layer F.Cu) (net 1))
 (segment (start 93.8295 69.4925) (end 92.583 69.4925) (width 1) (layer F.Cu) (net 1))
 (segment (start 103.0351 67.8307) (end 101.7868 69.079) (width 1) (layer F.Cu) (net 1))
 (segment (start 103.0351 64.4779) (end 103.0351 67.8307) (width 1) (layer F.Cu) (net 1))
 (segment (start 94.243 69.079) (end 93.8295 69.4925) (width 1) (layer F.Cu) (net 1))
 (segment (start 101.7868 69.079) (end 94.243 69.079) (width 1) (layer F.Cu) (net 1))
 (segment (start 101.7651 63.2079) (end 103.0351 64.4779) (width 1) (layer F.Cu) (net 1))
 (segment (start 101.7651 61.459) (end 101.7651 63.2079) (width 1) (layer F.Cu) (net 1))
 (segment (start 78.3148 53.5498) (end 78.359 53.594) (width 0.25) (layer F.Cu) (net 12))
 (segment (start 101.7651 53.6448) (end 101.7651 57.159) (width 2) (layer F.Cu) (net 12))
 (segment (start 55.88 67.31) (end 56.515 67.31) (width 0.25) (layer F.Cu) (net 11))
 (segment (start 56.515 67.31) (end 57.15 67.945) (width 0.25) (layer F.Cu) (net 11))
 (segment (start 87.6535 61.341) (end 87.6535 61.5715) (width 0.25) (layer F.Cu) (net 5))
 (segment (start 86.487 62.738) (end 86.487 63.946) (width 0.25) (layer F.Cu) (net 5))
 (segment (start 87.6535 61.5715) (end 86.487 62.738) (width 0.25) (layer F.Cu) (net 5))
 (segment (start 87.6535 61.341) (end 88.4285 60.566) (width 0.75) (layer F.Cu) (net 5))
 (segment (start 94.0811 58.6858) (end 94.107 58.7117) (width 2) (layer F.Cu) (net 5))
 (segment (start 93.1802 60.566) (end 94.107 59.6392) (width 0.75) (layer F.Cu) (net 5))
 (segment (start 91.3508 60.566) (end 93.1802 60.566) (width 0.75) (layer F.Cu) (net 5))
 (segment (start 94.107 59.6392) (end 94.107 58.7117) (width 1) (layer F.Cu) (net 5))
 (segment (start 94.107 60.566) (end 94.107 59.6392) (width 1) (layer F.Cu) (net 5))
 (segment (start 88.4285 60.566) (end 91.3508 60.566) (width 0.75) (layer F.Cu) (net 5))
 (segment (start 91.3508 60.566) (end 94.107 60.566) (width 0.75) (layer F.Cu) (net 5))
 (segment (start 93.2415 64.135) (end 94.996 64.135) (width 1) (layer F.Cu) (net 13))
 (segment (start 96.8883 66.0273) (end 94.996 64.135) (width 1) (layer F.Cu) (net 13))
 (segment (start 100.8126 66.0273) (end 96.8883 66.0273) (width 1) (layer F.Cu) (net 13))
 (segment (start 73.2028 69.215) (end 71.69101 69.215) (width 1) (layer F.Cu) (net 16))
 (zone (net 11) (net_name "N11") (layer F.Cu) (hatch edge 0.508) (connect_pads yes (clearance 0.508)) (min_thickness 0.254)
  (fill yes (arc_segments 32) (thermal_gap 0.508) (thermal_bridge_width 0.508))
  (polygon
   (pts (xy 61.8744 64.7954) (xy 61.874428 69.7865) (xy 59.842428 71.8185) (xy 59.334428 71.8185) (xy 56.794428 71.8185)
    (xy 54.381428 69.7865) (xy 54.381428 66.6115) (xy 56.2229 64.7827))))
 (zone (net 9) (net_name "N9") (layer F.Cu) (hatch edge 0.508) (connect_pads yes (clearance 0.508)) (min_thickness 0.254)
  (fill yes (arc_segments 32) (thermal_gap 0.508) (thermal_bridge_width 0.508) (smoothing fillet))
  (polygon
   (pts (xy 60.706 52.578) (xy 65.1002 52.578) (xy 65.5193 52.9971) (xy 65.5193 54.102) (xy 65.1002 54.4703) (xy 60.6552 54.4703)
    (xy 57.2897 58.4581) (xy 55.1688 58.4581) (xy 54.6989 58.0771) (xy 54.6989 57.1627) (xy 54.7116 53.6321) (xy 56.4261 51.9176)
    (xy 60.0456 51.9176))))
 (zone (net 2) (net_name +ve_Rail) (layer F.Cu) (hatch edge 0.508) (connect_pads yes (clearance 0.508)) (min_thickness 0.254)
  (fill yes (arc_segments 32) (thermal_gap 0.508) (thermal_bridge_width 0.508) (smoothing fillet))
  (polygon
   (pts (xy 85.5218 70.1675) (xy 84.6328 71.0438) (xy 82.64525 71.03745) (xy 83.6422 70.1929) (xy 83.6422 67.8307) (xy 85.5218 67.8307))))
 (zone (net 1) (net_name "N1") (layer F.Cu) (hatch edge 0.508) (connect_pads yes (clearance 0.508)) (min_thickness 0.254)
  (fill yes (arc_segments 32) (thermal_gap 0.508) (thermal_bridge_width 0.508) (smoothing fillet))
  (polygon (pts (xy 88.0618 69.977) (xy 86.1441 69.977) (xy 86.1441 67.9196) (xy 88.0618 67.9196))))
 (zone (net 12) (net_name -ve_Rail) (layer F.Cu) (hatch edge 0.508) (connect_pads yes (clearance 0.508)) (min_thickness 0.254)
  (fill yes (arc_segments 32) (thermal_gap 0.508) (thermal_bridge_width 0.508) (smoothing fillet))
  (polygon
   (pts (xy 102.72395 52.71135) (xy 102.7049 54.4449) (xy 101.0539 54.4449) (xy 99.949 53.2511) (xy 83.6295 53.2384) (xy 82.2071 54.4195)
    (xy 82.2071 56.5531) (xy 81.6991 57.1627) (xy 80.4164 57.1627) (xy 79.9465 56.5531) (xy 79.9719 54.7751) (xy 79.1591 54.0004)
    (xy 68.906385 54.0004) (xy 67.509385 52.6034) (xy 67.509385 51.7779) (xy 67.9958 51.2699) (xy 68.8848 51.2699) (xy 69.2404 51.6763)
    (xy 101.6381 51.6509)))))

